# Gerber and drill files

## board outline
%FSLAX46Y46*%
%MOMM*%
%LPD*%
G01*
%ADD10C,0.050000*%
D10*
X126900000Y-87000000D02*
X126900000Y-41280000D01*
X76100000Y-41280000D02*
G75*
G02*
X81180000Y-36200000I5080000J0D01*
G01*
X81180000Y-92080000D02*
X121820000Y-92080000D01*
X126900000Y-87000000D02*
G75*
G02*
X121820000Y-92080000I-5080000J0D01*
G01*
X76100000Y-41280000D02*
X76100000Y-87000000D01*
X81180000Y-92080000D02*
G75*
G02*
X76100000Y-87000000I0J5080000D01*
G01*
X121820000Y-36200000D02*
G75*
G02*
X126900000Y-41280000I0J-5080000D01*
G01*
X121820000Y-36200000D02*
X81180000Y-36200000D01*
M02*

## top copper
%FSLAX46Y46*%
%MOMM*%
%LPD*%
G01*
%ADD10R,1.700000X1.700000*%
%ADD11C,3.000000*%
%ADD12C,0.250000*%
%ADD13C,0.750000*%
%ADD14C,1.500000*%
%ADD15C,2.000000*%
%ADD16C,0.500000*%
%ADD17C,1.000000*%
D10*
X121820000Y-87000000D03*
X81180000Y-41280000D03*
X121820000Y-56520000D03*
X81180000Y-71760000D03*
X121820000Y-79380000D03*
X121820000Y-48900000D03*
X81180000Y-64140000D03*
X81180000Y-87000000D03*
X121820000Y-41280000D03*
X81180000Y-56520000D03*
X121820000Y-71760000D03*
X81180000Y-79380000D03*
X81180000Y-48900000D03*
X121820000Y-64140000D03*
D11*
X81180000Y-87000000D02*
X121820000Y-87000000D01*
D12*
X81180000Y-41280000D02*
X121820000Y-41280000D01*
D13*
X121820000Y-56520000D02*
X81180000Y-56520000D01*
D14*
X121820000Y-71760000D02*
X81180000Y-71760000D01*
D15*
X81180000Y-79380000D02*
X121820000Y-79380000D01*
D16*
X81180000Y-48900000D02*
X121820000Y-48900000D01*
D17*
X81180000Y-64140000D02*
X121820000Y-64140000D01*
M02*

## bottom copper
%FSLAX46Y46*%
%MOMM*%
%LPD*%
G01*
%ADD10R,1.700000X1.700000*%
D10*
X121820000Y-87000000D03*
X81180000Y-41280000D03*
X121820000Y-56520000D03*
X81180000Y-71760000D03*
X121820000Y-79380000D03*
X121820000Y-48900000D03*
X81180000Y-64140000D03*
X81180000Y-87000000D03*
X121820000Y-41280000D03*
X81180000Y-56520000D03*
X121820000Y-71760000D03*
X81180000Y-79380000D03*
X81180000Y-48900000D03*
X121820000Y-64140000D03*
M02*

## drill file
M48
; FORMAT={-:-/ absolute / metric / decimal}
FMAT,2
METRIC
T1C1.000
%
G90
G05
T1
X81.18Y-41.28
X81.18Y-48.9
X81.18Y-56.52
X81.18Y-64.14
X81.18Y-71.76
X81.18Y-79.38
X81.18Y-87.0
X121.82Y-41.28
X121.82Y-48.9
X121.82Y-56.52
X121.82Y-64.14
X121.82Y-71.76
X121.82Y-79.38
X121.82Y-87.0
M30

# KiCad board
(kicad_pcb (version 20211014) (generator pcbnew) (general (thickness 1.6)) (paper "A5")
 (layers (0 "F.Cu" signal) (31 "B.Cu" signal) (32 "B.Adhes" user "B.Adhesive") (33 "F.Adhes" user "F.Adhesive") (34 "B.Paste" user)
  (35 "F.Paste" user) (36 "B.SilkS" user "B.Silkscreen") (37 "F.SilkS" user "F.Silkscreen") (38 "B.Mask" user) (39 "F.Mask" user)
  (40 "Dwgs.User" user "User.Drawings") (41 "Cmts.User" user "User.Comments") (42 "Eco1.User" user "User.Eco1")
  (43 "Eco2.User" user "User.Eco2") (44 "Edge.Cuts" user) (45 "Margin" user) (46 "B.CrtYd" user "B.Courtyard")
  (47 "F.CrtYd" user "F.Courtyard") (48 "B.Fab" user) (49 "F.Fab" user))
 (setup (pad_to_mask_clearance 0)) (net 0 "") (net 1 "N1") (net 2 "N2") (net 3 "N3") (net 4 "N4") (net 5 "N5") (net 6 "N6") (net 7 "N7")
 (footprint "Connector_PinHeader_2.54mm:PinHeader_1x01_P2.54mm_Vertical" (layer "F.Cu") (at 121.82 87)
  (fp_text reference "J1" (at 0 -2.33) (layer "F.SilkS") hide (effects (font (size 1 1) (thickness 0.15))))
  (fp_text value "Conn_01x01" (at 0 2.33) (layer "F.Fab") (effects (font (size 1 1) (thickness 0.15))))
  (pad "1" thru_hole rect locked (at 0 0) (size 1.7 1.7) (drill 1) (layers *.Cu *.Mask) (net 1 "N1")))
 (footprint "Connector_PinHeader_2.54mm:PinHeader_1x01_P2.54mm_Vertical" (layer "F.Cu") (at 81.18 41.28)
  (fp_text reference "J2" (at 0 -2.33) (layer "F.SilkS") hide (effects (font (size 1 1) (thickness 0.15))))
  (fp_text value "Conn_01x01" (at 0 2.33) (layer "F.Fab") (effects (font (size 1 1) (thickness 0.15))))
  (pad "1" thru_hole rect locked (at 0 0) (size 1.7 1.7) (drill 1) (layers *.Cu *.Mask) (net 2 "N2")))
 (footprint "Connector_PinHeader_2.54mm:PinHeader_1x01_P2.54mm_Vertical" (layer "F.Cu") (at 121.82 56.52)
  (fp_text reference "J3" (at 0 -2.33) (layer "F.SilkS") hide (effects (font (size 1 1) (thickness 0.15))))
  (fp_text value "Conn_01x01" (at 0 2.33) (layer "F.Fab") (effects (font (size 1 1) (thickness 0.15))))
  (pad "1" thru_hole rect locked (at 0 0) (size 1.7 1.7) (drill 1) (layers *.Cu *.Mask) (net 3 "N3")))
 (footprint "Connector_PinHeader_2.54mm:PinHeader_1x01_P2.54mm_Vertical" (layer "F.Cu") (at 81.18 71.76)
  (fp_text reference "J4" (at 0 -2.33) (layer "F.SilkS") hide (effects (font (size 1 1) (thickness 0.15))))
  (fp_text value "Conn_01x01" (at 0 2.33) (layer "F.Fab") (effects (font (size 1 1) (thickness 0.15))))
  (pad "1" thru_hole rect locked (at 0 0) (size 1.7 1.7) (drill 1) (layers *.Cu *.Mask) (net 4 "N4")))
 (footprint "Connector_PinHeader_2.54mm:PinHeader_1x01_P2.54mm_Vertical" (layer "F.Cu") (at 121.82 79.38)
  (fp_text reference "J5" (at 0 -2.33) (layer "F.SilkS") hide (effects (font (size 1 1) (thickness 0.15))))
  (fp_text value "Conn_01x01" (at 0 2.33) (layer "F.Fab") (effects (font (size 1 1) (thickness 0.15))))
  (pad "1" thru_hole rect locked (at 0 0) (size 1.7 1.7) (drill 1) (layers *.Cu *.Mask) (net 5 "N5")))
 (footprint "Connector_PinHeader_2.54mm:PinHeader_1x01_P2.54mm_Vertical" (layer "F.Cu") (at 121.82 48.9)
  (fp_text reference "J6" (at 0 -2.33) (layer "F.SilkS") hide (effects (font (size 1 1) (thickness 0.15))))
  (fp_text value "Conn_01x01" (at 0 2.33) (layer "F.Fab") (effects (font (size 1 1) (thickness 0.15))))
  (pad "1" thru_hole rect locked (at 0 0) (size 1.7 1.7) (drill 1) (layers *.Cu *.Mask) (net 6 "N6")))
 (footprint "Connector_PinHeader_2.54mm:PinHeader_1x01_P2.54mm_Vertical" (layer "F.Cu") (at 81.18 64.14)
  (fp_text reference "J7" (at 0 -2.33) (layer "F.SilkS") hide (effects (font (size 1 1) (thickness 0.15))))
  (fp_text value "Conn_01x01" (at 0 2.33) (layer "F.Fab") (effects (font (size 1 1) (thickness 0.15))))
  (pad "1" thru_hole rect locked (at 0 0) (size 1.7 1.7) (drill 1) (layers *.Cu *.Mask) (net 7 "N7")))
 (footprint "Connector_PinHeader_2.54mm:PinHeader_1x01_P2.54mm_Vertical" (layer "F.Cu") (at 81.18 87)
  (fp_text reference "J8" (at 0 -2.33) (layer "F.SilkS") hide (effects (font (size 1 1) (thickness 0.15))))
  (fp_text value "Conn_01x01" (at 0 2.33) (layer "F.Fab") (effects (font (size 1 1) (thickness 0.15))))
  (pad "1" thru_hole rect locked (at 0 0) (size 1.7 1.7) (drill 1) (layers *.Cu *.Mask) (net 1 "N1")))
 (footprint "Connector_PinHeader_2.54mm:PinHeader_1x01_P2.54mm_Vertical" (layer "F.Cu") (at 121.82 41.28)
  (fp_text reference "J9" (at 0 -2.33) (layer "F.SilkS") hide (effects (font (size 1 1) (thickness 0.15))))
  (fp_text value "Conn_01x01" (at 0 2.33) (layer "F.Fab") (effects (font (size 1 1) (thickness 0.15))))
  (pad "1" thru_hole rect locked (at 0 0) (size 1.7 1.7) (drill 1) (layers *.Cu *.Mask) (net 2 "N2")))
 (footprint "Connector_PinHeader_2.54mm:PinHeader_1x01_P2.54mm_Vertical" (layer "F.Cu") (at 81.18 56.52)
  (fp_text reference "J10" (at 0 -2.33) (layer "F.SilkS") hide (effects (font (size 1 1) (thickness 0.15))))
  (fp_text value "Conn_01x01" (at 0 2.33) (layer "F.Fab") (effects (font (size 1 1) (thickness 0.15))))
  (pad "1" thru_hole rect locked (at 0 0) (size 1.7 1.7) (drill 1) (layers *.Cu *.Mask) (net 3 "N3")))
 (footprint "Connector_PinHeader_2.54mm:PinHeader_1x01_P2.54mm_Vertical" (layer "F.Cu") (at 121.82 71.76)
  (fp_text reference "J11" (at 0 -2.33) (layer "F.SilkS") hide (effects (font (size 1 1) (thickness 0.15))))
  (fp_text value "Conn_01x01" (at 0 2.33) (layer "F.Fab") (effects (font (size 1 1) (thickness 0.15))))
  (pad "1" thru_hole rect locked (at 0 0) (size 1.7 1.7) (drill 1) (layers *.Cu *.Mask) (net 4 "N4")))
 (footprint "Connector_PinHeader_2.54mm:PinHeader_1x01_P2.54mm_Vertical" (layer "F.Cu") (at 81.18 79.38)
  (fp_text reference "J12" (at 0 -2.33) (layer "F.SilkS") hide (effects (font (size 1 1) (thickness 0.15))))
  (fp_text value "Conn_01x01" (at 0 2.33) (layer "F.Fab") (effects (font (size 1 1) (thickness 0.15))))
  (pad "1" thru_hole rect locked (at 0 0) (size 1.7 1.7) (drill 1) (layers *.Cu *.Mask) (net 5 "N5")))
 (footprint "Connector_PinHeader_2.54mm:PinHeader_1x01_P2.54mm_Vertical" (layer "F.Cu") (at 81.18 48.9)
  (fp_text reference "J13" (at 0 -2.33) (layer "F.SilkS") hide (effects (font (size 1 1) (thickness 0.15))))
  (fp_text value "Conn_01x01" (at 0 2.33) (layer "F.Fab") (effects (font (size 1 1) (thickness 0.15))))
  (pad "1" thru_hole rect locked (at 0 0) (size 1.7 1.7) (drill 1) (layers *.Cu *.Mask) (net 6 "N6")))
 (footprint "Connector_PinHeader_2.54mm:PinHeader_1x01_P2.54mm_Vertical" (layer "F.Cu") (at 121.82 64.14)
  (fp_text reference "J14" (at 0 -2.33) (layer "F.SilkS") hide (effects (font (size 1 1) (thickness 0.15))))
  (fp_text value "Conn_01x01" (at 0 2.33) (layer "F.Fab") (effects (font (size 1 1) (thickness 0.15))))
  (pad "1" thru_hole rect locked (at 0 0) (size 1.7 1.7) (drill 1) (layers *.Cu *.Mask) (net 7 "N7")))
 (gr_line (start 126.9 87) (end 126.9 41.28) (layer "Edge.Cuts") (width 0.05))
 (gr_arc (start 76.1 41.28) (mid 77.587898 37.687898) (end 81.18 36.2) (layer "Edge.Cuts") (width 0.05))
 (gr_line (start 81.18 92.08) (end 121.82 92.08) (layer "Edge.Cuts") (width 0.05))
 (gr_arc (start 126.9 87) (mid 125.412102 90.592102) (end 121.82 92.08) (layer "Edge.Cuts") (width 0.05))
 (gr_line (start 76.1 41.28) (end 76.1 87) (layer "Edge.Cuts") (width 0.05))
 (gr_arc (start 81.18 92.08) (mid 77.587898 90.592102) (end 76.1 87) (layer "Edge.Cuts") (width 0.05))
 (gr_arc (start 121.82 36.2) (mid 125.412102 37.687898) (end 126.9 41.28) (layer "Edge.Cuts") (width 0.05))
 (gr_line (start 121.82 36.2) (end 81.18 36.2) (layer "Edge.Cuts") (width 0.05))
 (segment (start 81.18 87) (end 121.82 87) (width 3) (layer "F.Cu") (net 1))
 (segment (start 81.18 41.28) (end 121.82 41.28) (width 0.25) (layer "F.Cu") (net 2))
 (segment (start 121.82 56.52) (end 81.18 56.52) (width 0.75) (layer "F.Cu") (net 3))
 (segment (start 121.82 71.76) (end 81.18 71.76) (width 1.5) (layer "F.Cu") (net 4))
 (segment (start 81.18 79.38) (end 121.82 79.38) (width 2) (layer "F.Cu") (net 5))
 (segment (start 81.18 48.9) (end 121.82 48.9) (width 0.5) (layer "F.Cu") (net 6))
 (segment (start 81.18 64.14) (end 121.82 64.14) (width 1) (layer "F.Cu") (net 7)))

